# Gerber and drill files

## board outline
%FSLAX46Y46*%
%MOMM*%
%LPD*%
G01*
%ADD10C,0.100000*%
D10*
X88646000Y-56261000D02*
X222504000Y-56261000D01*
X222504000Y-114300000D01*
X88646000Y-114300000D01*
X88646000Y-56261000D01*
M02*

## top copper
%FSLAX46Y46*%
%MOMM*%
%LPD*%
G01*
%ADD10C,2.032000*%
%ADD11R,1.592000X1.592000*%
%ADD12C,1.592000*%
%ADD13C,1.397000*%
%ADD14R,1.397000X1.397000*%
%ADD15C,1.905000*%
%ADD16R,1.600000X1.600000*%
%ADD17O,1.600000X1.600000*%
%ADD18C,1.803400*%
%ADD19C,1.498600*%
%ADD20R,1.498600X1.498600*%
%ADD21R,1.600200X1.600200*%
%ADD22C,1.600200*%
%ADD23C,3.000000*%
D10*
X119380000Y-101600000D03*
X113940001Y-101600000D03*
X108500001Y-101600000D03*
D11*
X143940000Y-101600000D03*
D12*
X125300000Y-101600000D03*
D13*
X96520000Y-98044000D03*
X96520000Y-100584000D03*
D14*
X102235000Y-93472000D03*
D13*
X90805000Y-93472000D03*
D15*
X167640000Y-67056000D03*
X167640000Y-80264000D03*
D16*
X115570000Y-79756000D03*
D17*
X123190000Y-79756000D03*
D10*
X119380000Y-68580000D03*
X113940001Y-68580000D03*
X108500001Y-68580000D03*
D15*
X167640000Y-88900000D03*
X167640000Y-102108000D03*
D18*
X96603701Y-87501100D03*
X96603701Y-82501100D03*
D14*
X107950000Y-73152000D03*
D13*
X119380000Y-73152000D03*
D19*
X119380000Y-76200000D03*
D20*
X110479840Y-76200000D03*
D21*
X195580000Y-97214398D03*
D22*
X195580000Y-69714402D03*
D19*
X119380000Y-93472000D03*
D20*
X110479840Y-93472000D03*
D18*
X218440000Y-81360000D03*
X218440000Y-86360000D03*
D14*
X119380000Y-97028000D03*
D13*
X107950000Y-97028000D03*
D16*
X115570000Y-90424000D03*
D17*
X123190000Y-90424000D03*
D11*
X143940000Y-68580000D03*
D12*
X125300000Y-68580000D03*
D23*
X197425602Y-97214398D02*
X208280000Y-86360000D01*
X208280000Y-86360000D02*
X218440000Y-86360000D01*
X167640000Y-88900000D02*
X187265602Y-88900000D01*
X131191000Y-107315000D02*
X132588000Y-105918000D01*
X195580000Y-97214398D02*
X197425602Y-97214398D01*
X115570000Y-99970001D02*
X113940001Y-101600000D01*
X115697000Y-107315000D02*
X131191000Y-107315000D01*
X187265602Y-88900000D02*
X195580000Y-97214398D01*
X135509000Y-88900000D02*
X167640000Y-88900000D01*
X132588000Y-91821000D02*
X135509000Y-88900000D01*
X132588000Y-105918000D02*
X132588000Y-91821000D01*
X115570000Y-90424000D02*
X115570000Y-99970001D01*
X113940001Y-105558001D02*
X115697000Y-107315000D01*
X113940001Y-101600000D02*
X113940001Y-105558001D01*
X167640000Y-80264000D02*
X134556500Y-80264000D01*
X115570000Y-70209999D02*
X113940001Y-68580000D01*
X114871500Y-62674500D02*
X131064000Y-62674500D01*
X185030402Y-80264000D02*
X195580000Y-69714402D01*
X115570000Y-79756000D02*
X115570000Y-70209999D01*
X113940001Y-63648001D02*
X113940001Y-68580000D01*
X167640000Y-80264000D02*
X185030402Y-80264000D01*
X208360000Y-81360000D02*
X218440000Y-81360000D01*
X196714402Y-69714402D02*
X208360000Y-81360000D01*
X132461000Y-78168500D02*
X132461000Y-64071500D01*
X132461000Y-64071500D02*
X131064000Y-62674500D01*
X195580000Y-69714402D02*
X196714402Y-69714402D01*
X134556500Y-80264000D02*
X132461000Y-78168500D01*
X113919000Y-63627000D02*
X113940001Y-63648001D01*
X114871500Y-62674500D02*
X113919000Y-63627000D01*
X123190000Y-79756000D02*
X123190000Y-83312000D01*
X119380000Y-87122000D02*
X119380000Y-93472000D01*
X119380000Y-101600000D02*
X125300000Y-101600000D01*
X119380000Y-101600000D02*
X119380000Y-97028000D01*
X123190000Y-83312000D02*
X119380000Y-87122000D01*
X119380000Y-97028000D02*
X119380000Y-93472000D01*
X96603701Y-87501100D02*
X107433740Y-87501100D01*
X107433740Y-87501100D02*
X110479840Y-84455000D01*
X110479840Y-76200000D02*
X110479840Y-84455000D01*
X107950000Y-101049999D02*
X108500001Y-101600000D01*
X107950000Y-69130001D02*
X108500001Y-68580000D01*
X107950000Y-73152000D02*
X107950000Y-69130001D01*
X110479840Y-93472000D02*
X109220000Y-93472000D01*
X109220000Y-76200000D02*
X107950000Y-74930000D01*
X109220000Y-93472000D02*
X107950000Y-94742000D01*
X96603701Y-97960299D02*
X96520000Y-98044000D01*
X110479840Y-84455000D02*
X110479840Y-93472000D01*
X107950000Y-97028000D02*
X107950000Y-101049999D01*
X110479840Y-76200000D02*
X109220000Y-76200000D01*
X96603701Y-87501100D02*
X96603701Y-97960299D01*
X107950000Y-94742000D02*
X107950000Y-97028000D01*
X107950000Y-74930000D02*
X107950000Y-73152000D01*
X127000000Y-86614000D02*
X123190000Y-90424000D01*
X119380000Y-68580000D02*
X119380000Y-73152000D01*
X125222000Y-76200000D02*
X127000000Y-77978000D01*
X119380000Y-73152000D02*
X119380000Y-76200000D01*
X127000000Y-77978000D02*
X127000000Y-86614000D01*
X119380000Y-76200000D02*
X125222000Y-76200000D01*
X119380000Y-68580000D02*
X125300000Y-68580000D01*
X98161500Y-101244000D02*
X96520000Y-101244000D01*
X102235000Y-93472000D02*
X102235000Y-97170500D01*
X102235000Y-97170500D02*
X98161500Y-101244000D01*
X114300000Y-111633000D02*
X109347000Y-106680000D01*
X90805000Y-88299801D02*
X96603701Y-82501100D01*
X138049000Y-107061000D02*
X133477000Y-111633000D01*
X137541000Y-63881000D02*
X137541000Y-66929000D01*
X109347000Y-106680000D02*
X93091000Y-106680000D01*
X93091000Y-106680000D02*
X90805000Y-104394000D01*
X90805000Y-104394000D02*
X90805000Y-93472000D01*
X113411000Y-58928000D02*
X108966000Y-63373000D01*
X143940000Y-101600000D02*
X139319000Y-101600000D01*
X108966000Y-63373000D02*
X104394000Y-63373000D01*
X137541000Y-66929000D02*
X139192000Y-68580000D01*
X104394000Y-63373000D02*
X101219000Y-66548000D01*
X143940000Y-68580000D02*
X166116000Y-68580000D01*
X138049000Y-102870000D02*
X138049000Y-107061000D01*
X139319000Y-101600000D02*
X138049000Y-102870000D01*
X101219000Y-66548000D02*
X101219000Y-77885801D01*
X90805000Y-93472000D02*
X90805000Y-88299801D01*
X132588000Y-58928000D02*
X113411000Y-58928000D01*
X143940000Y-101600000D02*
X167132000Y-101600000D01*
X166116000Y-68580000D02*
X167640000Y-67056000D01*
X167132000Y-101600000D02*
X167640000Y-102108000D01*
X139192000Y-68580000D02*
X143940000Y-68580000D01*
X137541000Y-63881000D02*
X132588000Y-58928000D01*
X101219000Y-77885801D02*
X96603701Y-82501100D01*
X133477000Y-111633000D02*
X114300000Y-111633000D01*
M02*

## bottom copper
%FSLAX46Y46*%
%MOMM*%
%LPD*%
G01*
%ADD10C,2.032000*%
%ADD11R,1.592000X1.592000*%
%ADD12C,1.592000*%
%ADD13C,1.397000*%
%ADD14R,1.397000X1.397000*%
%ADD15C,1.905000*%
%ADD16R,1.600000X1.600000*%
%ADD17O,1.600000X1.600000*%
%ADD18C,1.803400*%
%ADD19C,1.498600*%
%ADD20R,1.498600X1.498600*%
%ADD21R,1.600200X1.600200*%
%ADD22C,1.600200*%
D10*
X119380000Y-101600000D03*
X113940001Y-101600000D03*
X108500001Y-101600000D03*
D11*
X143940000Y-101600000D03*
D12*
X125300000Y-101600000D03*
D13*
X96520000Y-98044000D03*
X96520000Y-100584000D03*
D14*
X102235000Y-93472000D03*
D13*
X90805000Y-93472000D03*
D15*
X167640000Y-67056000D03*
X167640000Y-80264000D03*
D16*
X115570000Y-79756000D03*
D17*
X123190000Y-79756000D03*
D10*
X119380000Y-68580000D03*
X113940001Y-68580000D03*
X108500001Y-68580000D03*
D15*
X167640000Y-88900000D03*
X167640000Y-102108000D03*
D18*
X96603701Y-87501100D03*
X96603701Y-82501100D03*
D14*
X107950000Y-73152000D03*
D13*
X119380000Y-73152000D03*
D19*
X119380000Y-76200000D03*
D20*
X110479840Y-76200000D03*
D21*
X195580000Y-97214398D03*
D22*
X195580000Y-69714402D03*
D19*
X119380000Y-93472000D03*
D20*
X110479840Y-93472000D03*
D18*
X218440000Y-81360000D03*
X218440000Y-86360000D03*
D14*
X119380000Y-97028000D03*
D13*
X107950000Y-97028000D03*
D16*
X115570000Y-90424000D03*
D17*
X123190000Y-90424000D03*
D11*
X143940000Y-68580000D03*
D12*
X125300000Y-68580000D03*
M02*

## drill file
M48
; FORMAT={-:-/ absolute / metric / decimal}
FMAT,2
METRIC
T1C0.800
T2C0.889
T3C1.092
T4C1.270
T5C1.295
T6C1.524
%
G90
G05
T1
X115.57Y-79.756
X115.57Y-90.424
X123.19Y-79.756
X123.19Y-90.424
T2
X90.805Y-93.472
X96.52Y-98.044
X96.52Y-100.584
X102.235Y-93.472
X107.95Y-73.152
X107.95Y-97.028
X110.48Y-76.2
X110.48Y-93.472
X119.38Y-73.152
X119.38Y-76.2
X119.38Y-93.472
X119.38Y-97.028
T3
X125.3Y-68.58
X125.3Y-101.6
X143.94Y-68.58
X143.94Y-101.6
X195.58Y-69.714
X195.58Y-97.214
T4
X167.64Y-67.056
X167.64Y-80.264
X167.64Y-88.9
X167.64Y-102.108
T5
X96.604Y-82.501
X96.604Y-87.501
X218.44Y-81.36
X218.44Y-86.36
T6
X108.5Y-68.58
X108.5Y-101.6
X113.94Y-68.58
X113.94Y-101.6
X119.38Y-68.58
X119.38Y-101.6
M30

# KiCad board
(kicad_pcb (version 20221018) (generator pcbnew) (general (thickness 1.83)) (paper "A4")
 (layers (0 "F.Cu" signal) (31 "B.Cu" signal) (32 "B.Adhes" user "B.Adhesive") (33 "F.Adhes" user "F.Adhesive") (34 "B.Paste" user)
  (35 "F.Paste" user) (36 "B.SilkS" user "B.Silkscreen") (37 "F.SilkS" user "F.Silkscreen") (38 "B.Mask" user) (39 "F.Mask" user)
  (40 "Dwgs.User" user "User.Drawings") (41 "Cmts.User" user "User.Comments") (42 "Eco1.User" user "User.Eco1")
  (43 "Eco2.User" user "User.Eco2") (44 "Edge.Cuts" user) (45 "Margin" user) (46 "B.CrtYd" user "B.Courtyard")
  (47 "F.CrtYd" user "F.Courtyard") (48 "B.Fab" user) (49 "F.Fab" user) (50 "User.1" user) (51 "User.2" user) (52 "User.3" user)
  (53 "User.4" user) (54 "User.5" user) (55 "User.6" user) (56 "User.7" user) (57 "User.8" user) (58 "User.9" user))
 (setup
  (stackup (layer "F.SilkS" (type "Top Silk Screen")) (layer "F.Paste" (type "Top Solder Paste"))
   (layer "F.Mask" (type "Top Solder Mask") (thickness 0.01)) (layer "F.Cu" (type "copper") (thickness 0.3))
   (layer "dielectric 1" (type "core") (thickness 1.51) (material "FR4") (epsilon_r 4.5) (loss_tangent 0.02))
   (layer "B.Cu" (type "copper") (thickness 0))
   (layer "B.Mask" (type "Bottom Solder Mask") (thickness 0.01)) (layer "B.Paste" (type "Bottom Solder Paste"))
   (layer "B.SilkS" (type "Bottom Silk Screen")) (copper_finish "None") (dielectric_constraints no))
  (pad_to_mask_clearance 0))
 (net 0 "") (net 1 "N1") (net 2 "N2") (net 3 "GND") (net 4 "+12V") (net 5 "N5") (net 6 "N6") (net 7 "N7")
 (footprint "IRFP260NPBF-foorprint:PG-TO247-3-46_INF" (layer "F.Cu") (at 119.38 101.6 180)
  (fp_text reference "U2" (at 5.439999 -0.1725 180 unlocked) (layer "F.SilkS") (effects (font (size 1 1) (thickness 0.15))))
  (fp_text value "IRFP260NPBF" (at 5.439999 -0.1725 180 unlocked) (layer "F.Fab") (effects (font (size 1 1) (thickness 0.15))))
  (pad "1" thru_hole circle (at 0 0 180) (size 2.032 2.032) (drill 1.524) (layers "*.Cu" "*.Mask") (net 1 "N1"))
  (pad "2" thru_hole circle (at 5.439999 0 180) (size 2.032 2.032) (drill 1.524) (layers "*.Cu" "*.Mask") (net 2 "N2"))
  (pad "3" thru_hole circle (at 10.879999 0 180) (size 2.032 2.032) (drill 1.524) (layers "*.Cu" "*.Mask") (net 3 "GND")))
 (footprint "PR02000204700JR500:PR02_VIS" (layer "F.Cu") (at 143.939999 101.6 180)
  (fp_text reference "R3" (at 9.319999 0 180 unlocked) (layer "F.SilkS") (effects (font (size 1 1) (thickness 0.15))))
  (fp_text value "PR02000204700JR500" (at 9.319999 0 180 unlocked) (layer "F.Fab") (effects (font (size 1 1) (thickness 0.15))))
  (pad "1" thru_hole rect (at -0.000001 0 180) (size 1.592 1.592) (drill 1.0922) (layers "*.Cu" "*.Mask") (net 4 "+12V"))
  (pad "2" thru_hole circle (at 18.639999 0 180) (size 1.592 1.592) (drill 1.0922) (layers "*.Cu" "*.Mask") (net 1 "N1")))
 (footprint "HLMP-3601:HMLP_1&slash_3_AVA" (layer "F.Cu") (at 96.52 98.044 -90)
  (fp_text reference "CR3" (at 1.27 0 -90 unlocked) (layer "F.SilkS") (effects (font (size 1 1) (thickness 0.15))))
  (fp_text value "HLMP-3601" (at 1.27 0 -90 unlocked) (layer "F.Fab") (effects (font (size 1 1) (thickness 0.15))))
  (pad "1" thru_hole circle (at 0 0 270) (size 1.397 1.397) (drill 0.889) (layers "*.Cu" "*.Mask") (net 3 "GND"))
  (pad "2" thru_hole circle (at 2.54 0 270) (size 1.397 1.397) (drill 0.889) (layers "*.Cu" "*.Mask") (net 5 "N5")))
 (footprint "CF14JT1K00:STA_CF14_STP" (layer "F.Cu") (at 102.235 93.472 180)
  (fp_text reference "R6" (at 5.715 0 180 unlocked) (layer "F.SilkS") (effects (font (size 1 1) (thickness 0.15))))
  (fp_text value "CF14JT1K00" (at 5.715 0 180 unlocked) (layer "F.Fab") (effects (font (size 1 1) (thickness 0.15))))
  (pad "1" thru_hole rect (at 0 0 180) (size 1.397 1.397) (drill 0.889) (layers "*.Cu" "*.Mask") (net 5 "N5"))
  (pad "2" thru_hole circle (at 11.43 0 180) (size 1.397 1.397) (drill 0.889) (layers "*.Cu" "*.Mask") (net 4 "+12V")))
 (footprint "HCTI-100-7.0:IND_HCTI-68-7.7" (layer "F.Cu") (at 167.64 73.66 -90)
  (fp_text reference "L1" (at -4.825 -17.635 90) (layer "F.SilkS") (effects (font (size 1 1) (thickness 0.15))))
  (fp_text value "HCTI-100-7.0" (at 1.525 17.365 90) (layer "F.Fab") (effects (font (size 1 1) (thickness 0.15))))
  (pad "1" thru_hole circle (at -6.604 0 270) (size 1.905 1.905) (drill 1.27) (layers "*.Cu" "*.Mask") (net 4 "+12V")
   (solder_mask_margin 0.102))
  (pad "2" thru_hole circle (at 6.604 0 270) (size 1.905 1.905) (drill 1.27) (layers "*.Cu" "*.Mask") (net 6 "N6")
   (solder_mask_margin 0.102)))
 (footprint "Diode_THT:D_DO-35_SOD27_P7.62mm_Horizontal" (layer "F.Cu") (at 115.57 79.756)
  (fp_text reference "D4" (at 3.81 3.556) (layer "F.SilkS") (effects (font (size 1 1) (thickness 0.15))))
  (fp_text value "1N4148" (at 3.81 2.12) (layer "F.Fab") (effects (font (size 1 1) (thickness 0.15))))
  (pad "1" thru_hole rect (at 0 0) (size 1.6 1.6) (drill 0.8) (layers "*.Cu" "*.Mask") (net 6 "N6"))
  (pad "2" thru_hole oval (at 7.62 0) (size 1.6 1.6) (drill 0.8) (layers "*.Cu" "*.Mask") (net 1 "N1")))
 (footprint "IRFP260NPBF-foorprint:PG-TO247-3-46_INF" (layer "F.Cu") (at 119.38 68.58 180)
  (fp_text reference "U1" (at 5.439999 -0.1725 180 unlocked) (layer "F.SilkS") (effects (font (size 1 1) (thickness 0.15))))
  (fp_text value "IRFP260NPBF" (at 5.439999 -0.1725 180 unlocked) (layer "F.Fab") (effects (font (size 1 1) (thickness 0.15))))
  (pad "1" thru_hole circle (at 0 0 180) (size 2.032 2.032) (drill 1.524) (layers "*.Cu" "*.Mask") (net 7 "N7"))
  (pad "2" thru_hole circle (at 5.439999 0 180) (size 2.032 2.032) (drill 1.524) (layers "*.Cu" "*.Mask") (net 6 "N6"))
  (pad "3" thru_hole circle (at 10.879999 0 180) (size 2.032 2.032) (drill 1.524) (layers "*.Cu" "*.Mask") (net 3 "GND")))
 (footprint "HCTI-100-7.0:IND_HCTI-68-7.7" (layer "F.Cu") (at 167.64 95.504 -90)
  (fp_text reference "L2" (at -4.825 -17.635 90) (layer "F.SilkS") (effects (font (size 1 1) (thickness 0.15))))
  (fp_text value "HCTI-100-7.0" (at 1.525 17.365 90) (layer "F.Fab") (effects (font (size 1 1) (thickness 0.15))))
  (pad "1" thru_hole circle (at -6.604 0 270) (size 1.905 1.905) (drill 1.27) (layers "*.Cu" "*.Mask") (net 2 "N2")
   (solder_mask_margin 0.102))
  (pad "2" thru_hole circle (at 6.604 0 270) (size 1.905 1.905) (drill 1.27) (layers "*.Cu" "*.Mask") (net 4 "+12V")
   (solder_mask_margin 0.102)))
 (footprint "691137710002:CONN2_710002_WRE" (layer "F.Cu") (at 96.603701 87.5011 90)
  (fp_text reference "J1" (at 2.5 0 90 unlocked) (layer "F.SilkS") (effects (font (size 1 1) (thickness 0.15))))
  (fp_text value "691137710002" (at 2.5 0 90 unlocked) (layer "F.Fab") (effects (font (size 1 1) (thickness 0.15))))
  (pad "1" thru_hole circle (at 0 0 90) (size 1.8034 1.8034) (drill 1.2954) (layers "*.Cu" "*.Mask") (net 3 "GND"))
  (pad "2" thru_hole circle (at 5 0 90) (size 1.8034 1.8034) (drill 1.2954) (layers "*.Cu" "*.Mask") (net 4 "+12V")))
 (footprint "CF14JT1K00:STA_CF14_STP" (layer "F.Cu") (at 107.95 73.152)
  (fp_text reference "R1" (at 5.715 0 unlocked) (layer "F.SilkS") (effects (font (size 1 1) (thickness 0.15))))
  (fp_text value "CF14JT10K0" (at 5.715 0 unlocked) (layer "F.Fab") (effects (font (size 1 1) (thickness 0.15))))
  (pad "1" thru_hole rect (at 0 0) (size 1.397 1.397) (drill 0.889) (layers "*.Cu" "*.Mask") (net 3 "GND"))
  (pad "2" thru_hole circle (at 11.43 0) (size 1.397 1.397) (drill 0.889) (layers "*.Cu" "*.Mask") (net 7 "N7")))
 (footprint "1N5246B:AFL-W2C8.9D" (layer "F.Cu") (at 110.47984 76.2 180)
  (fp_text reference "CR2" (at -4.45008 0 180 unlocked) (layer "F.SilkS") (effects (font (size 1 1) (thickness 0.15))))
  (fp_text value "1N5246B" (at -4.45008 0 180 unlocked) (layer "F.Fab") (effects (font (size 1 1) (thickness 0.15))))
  (pad "1" thru_hole circle (at -8.90016 0 180) (size 1.4986 1.4986) (drill 0.889) (layers "*.Cu" "*.Mask") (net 7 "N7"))
  (pad "2" thru_hole rect (at 0 0 180) (size 1.4986 1.4986) (drill 0.889) (layers "*.Cu" "*.Mask") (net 3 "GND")))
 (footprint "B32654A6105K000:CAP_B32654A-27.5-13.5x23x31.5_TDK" (layer "F.Cu") (at 195.58 97.214398 90)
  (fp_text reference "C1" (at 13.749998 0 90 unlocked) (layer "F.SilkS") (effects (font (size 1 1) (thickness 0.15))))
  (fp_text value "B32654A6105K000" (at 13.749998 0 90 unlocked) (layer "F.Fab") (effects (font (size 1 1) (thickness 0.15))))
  (pad "1" thru_hole rect (at 0 0 90) (size 1.6002 1.6002) (drill 1.0922) (layers "*.Cu" "*.Mask") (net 2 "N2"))
  (pad "2" thru_hole circle (at 27.499996 0 90) (size 1.6002 1.6002) (drill 1.0922) (layers "*.Cu" "*.Mask") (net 6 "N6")))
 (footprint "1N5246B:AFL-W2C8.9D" (layer "F.Cu") (at 110.47984 93.472 180)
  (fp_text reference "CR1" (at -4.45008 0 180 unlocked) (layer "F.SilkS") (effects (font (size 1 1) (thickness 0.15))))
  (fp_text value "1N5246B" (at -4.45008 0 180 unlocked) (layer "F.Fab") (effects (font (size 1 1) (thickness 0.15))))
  (pad "1" thru_hole circle (at -8.90016 0 180) (size 1.4986 1.4986) (drill 0.889) (layers "*.Cu" "*.Mask") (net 1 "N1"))
  (pad "2" thru_hole rect (at 0 0 180) (size 1.4986 1.4986) (drill 0.889) (layers "*.Cu" "*.Mask") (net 3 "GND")))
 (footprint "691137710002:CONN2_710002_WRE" (layer "F.Cu") (at 218.44 81.36 -90)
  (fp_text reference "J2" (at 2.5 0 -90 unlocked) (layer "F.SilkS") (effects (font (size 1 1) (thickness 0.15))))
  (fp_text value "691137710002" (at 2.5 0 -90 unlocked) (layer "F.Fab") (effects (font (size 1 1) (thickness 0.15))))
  (pad "1" thru_hole circle (at 0 0 270) (size 1.8034 1.8034) (drill 1.2954) (layers "*.Cu" "*.Mask") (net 6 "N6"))
  (pad "2" thru_hole circle (at 5 0 270) (size 1.8034 1.8034) (drill 1.2954) (layers "*.Cu" "*.Mask") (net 2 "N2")))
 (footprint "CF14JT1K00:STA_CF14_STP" (layer "F.Cu") (at 119.38 97.028 180)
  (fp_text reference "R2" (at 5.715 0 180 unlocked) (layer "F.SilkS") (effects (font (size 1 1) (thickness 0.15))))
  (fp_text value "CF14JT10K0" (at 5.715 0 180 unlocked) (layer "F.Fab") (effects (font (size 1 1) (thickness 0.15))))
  (pad "1" thru_hole rect (at 0 0 180) (size 1.397 1.397) (drill 0.889) (layers "*.Cu" "*.Mask") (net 1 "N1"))
  (pad "2" thru_hole circle (at 11.43 0 180) (size 1.397 1.397) (drill 0.889) (layers "*.Cu" "*.Mask") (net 3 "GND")))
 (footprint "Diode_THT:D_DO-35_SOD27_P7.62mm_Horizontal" (layer "F.Cu") (at 115.57 90.424)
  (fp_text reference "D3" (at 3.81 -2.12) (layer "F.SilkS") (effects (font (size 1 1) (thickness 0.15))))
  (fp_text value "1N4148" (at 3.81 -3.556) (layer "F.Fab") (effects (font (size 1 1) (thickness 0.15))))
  (pad "1" thru_hole rect (at 0 0) (size 1.6 1.6) (drill 0.8) (layers "*.Cu" "*.Mask") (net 2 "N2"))
  (pad "2" thru_hole oval (at 7.62 0) (size 1.6 1.6) (drill 0.8) (layers "*.Cu" "*.Mask") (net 7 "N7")))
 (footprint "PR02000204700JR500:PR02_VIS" (layer "F.Cu") (at 143.939999 68.58 180)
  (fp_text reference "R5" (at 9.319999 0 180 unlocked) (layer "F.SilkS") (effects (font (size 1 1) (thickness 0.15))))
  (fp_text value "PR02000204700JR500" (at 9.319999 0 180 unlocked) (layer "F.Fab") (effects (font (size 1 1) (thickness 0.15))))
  (pad "1" thru_hole rect (at -0.000001 0 180) (size 1.592 1.592) (drill 1.0922) (layers "*.Cu" "*.Mask") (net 4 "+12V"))
  (pad "2" thru_hole circle (at 18.639999 0 180) (size 1.592 1.592) (drill 1.0922) (layers "*.Cu" "*.Mask") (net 7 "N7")))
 (gr_rect (start 88.646 56.261) (end 222.504 114.3) (stroke (width 0.1) (type default)) (fill none) (layer "Edge.Cuts"))
 (segment (start 197.425602 97.214398) (end 208.28 86.36) (width 3) (layer "F.Cu") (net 2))
 (segment (start 208.28 86.36) (end 218.44 86.36) (width 3) (layer "F.Cu") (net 2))
 (segment (start 167.64 88.9) (end 187.265602 88.9) (width 3) (layer "F.Cu") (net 2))
 (segment (start 131.191 107.315) (end 132.588 105.918) (width 3) (layer "F.Cu") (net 2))
 (segment (start 195.58 97.214398) (end 197.425602 97.214398) (width 3) (layer "F.Cu") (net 2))
 (segment (start 115.57 99.970001) (end 113.940001 101.6) (width 3) (layer "F.Cu") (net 2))
 (segment (start 115.697 107.315) (end 131.191 107.315) (width 3) (layer "F.Cu") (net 2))
 (segment (start 187.265602 88.9) (end 195.58 97.214398) (width 3) (layer "F.Cu") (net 2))
 (segment (start 135.509 88.9) (end 167.64 88.9) (width 3) (layer "F.Cu") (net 2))
 (segment (start 132.588 91.821) (end 135.509 88.9) (width 3) (layer "F.Cu") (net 2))
 (segment (start 132.588 105.918) (end 132.588 91.821) (width 3) (layer "F.Cu") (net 2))
 (segment (start 115.57 90.424) (end 115.57 99.970001) (width 3) (layer "F.Cu") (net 2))
 (segment (start 113.940001 105.558001) (end 115.697 107.315) (width 3) (layer "F.Cu") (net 2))
 (segment (start 113.940001 101.6) (end 113.940001 105.558001) (width 3) (layer "F.Cu") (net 2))
 (segment (start 167.64 80.264) (end 134.5565 80.264) (width 3) (layer "F.Cu") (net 6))
 (segment (start 115.57 70.209999) (end 113.940001 68.58) (width 3) (layer "F.Cu") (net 6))
 (segment (start 114.8715 62.6745) (end 131.064 62.6745) (width 3) (layer "F.Cu") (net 6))
 (segment (start 185.030402 80.264) (end 195.58 69.714402) (width 3) (layer "F.Cu") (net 6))
 (segment (start 115.57 79.756) (end 115.57 70.209999) (width 3) (layer "F.Cu") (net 6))
 (segment (start 113.940001 63.648001) (end 113.940001 68.58) (width 3) (layer "F.Cu") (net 6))
 (segment (start 167.64 80.264) (end 185.030402 80.264) (width 3) (layer "F.Cu") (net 6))
 (segment (start 208.36 81.36) (end 218.44 81.36) (width 3) (layer "F.Cu") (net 6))
 (segment (start 196.714402 69.714402) (end 208.36 81.36) (width 3) (layer "F.Cu") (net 6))
 (segment (start 132.461 78.1685) (end 132.461 64.0715) (width 3) (layer "F.Cu") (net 6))
 (segment (start 132.461 64.0715) (end 131.064 62.6745) (width 3) (layer "F.Cu") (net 6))
 (segment (start 195.58 69.714402) (end 196.714402 69.714402) (width 3) (layer "F.Cu") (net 6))
 (segment (start 134.5565 80.264) (end 132.461 78.1685) (width 3) (layer "F.Cu") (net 6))
 (segment (start 113.919 63.627) (end 113.940001 63.648001) (width 3) (layer "F.Cu") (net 6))
 (segment (start 114.8715 62.6745) (end 113.919 63.627) (width 3) (layer "F.Cu") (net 6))
 (segment (start 123.19 79.756) (end 123.19 83.312) (width 3) (layer "F.Cu") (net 1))
 (segment (start 119.38 87.122) (end 119.38 93.472) (width 3) (layer "F.Cu") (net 1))
 (segment (start 119.38 101.6) (end 125.3 101.6) (width 3) (layer "F.Cu") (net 1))
 (segment (start 119.38 101.6) (end 119.38 97.028) (width 3) (layer "F.Cu") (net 1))
 (segment (start 123.19 83.312) (end 119.38 87.122) (width 3) (layer "F.Cu") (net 1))
 (segment (start 119.38 97.028) (end 119.38 93.472) (width 3) (layer "F.Cu") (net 1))
 (segment (start 96.603701 87.5011) (end 107.43374 87.5011) (width 3) (layer "F.Cu") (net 3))
 (segment (start 107.43374 87.5011) (end 110.47984 84.455) (width 3) (layer "F.Cu") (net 3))
 (segment (start 110.47984 76.2) (end 110.47984 84.455) (width 3) (layer "F.Cu") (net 3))
 (segment (start 107.95 101.049999) (end 108.500001 101.6) (width 3) (layer "F.Cu") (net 3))
 (segment (start 107.95 69.130001) (end 108.500001 68.58) (width 3) (layer "F.Cu") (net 3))
 (segment (start 107.95 73.152) (end 107.95 69.130001) (width 3) (layer "F.Cu") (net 3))
 (segment (start 110.47984 93.472) (end 109.22 93.472) (width 3) (layer "F.Cu") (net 3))
 (segment (start 109.22 76.2) (end 107.95 74.93) (width 3) (layer "F.Cu") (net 3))
 (segment (start 109.22 93.472) (end 107.95 94.742) (width 3) (layer "F.Cu") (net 3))
 (segment (start 96.603701 97.960299) (end 96.52 98.044) (width 3) (layer "F.Cu") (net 3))
 (segment (start 110.47984 84.455) (end 110.47984 93.472) (width 3) (layer "F.Cu") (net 3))
 (segment (start 107.95 97.028) (end 107.95 101.049999) (width 3) (layer "F.Cu") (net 3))
 (segment (start 110.47984 76.2) (end 109.22 76.2) (width 3) (layer "F.Cu") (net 3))
 (segment (start 96.603701 87.5011) (end 96.603701 97.960299) (width 3) (layer "F.Cu") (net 3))
 (segment (start 107.95 94.742) (end 107.95 97.028) (width 3) (layer "F.Cu") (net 3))
 (segment (start 107.95 74.93) (end 107.95 73.152) (width 3) (layer "F.Cu") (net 3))
 (segment (start 127 86.614) (end 123.19 90.424) (width 3) (layer "F.Cu") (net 7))
 (segment (start 119.38 68.58) (end 119.38 73.152) (width 3) (layer "F.Cu") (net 7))
 (segment (start 125.222 76.2) (end 127 77.978) (width 3) (layer "F.Cu") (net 7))
 (segment (start 119.38 73.152) (end 119.38 76.2) (width 3) (layer "F.Cu") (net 7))
 (segment (start 127 77.978) (end 127 86.614) (width 3) (layer "F.Cu") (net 7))
 (segment (start 119.38 76.2) (end 125.222 76.2) (width 3) (layer "F.Cu") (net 7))
 (segment (start 119.38 68.58) (end 125.3 68.58) (width 3) (layer "F.Cu") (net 7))
 (segment (start 98.1615 101.244) (end 96.52 101.244) (width 3) (layer "F.Cu") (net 5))
 (segment (start 102.235 93.472) (end 102.235 97.1705) (width 3) (layer "F.Cu") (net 5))
 (segment (start 102.235 97.1705) (end 98.1615 101.244) (width 3) (layer "F.Cu") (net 5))
 (segment (start 114.3 111.633) (end 109.347 106.68) (width 3) (layer "F.Cu") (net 4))
 (segment (start 90.805 88.299801) (end 96.603701 82.5011) (width 3) (layer "F.Cu") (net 4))
 (segment (start 138.049 107.061) (end 133.477 111.633) (width 3) (layer "F.Cu") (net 4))
 (segment (start 137.541 63.881) (end 137.541 66.929) (width 3) (layer "F.Cu") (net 4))
 (segment (start 109.347 106.68) (end 93.091 106.68) (width 3) (layer "F.Cu") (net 4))
 (segment (start 93.091 106.68) (end 90.805 104.394) (width 3) (layer "F.Cu") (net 4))
 (segment (start 90.805 104.394) (end 90.805 93.472) (width 3) (layer "F.Cu") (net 4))
 (segment (start 113.411 58.928) (end 108.966 63.373) (width 3) (layer "F.Cu") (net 4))
 (segment (start 143.94 101.6) (end 139.319 101.6) (width 3) (layer "F.Cu") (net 4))
 (segment (start 108.966 63.373) (end 104.394 63.373) (width 3) (layer "F.Cu") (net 4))
 (segment (start 137.541 66.929) (end 139.192 68.58) (width 3) (layer "F.Cu") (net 4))
 (segment (start 104.394 63.373) (end 101.219 66.548) (width 3) (layer "F.Cu") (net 4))
 (segment (start 143.94 68.58) (end 166.116 68.58) (width 3) (layer "F.Cu") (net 4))
 (segment (start 138.049 102.87) (end 138.049 107.061) (width 3) (layer "F.Cu") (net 4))
 (segment (start 139.319 101.6) (end 138.049 102.87) (width 3) (layer "F.Cu") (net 4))
 (segment (start 101.219 66.548) (end 101.219 77.885801) (width 3) (layer "F.Cu") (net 4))
 (segment (start 90.805 93.472) (end 90.805 88.299801) (width 3) (layer "F.Cu") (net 4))
 (segment (start 132.588 58.928) (end 113.411 58.928) (width 3) (layer "F.Cu") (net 4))
 (segment (start 143.94 101.6) (end 167.132 101.6) (width 3) (layer "F.Cu") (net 4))
 (segment (start 166.116 68.58) (end 167.64 67.056) (width 3) (layer "F.Cu") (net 4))
 (segment (start 167.132 101.6) (end 167.64 102.108) (width 3) (layer "F.Cu") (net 4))
 (segment (start 139.192 68.58) (end 143.94 68.58) (width 3) (layer "F.Cu") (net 4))
 (segment (start 137.541 63.881) (end 132.588 58.928) (width 3) (layer "F.Cu") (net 4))
 (segment (start 101.219 77.885801) (end 96.603701 82.5011) (width 3) (layer "F.Cu") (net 4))
 (segment (start 133.477 111.633) (end 114.3 111.633) (width 3) (layer "F.Cu") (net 4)))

